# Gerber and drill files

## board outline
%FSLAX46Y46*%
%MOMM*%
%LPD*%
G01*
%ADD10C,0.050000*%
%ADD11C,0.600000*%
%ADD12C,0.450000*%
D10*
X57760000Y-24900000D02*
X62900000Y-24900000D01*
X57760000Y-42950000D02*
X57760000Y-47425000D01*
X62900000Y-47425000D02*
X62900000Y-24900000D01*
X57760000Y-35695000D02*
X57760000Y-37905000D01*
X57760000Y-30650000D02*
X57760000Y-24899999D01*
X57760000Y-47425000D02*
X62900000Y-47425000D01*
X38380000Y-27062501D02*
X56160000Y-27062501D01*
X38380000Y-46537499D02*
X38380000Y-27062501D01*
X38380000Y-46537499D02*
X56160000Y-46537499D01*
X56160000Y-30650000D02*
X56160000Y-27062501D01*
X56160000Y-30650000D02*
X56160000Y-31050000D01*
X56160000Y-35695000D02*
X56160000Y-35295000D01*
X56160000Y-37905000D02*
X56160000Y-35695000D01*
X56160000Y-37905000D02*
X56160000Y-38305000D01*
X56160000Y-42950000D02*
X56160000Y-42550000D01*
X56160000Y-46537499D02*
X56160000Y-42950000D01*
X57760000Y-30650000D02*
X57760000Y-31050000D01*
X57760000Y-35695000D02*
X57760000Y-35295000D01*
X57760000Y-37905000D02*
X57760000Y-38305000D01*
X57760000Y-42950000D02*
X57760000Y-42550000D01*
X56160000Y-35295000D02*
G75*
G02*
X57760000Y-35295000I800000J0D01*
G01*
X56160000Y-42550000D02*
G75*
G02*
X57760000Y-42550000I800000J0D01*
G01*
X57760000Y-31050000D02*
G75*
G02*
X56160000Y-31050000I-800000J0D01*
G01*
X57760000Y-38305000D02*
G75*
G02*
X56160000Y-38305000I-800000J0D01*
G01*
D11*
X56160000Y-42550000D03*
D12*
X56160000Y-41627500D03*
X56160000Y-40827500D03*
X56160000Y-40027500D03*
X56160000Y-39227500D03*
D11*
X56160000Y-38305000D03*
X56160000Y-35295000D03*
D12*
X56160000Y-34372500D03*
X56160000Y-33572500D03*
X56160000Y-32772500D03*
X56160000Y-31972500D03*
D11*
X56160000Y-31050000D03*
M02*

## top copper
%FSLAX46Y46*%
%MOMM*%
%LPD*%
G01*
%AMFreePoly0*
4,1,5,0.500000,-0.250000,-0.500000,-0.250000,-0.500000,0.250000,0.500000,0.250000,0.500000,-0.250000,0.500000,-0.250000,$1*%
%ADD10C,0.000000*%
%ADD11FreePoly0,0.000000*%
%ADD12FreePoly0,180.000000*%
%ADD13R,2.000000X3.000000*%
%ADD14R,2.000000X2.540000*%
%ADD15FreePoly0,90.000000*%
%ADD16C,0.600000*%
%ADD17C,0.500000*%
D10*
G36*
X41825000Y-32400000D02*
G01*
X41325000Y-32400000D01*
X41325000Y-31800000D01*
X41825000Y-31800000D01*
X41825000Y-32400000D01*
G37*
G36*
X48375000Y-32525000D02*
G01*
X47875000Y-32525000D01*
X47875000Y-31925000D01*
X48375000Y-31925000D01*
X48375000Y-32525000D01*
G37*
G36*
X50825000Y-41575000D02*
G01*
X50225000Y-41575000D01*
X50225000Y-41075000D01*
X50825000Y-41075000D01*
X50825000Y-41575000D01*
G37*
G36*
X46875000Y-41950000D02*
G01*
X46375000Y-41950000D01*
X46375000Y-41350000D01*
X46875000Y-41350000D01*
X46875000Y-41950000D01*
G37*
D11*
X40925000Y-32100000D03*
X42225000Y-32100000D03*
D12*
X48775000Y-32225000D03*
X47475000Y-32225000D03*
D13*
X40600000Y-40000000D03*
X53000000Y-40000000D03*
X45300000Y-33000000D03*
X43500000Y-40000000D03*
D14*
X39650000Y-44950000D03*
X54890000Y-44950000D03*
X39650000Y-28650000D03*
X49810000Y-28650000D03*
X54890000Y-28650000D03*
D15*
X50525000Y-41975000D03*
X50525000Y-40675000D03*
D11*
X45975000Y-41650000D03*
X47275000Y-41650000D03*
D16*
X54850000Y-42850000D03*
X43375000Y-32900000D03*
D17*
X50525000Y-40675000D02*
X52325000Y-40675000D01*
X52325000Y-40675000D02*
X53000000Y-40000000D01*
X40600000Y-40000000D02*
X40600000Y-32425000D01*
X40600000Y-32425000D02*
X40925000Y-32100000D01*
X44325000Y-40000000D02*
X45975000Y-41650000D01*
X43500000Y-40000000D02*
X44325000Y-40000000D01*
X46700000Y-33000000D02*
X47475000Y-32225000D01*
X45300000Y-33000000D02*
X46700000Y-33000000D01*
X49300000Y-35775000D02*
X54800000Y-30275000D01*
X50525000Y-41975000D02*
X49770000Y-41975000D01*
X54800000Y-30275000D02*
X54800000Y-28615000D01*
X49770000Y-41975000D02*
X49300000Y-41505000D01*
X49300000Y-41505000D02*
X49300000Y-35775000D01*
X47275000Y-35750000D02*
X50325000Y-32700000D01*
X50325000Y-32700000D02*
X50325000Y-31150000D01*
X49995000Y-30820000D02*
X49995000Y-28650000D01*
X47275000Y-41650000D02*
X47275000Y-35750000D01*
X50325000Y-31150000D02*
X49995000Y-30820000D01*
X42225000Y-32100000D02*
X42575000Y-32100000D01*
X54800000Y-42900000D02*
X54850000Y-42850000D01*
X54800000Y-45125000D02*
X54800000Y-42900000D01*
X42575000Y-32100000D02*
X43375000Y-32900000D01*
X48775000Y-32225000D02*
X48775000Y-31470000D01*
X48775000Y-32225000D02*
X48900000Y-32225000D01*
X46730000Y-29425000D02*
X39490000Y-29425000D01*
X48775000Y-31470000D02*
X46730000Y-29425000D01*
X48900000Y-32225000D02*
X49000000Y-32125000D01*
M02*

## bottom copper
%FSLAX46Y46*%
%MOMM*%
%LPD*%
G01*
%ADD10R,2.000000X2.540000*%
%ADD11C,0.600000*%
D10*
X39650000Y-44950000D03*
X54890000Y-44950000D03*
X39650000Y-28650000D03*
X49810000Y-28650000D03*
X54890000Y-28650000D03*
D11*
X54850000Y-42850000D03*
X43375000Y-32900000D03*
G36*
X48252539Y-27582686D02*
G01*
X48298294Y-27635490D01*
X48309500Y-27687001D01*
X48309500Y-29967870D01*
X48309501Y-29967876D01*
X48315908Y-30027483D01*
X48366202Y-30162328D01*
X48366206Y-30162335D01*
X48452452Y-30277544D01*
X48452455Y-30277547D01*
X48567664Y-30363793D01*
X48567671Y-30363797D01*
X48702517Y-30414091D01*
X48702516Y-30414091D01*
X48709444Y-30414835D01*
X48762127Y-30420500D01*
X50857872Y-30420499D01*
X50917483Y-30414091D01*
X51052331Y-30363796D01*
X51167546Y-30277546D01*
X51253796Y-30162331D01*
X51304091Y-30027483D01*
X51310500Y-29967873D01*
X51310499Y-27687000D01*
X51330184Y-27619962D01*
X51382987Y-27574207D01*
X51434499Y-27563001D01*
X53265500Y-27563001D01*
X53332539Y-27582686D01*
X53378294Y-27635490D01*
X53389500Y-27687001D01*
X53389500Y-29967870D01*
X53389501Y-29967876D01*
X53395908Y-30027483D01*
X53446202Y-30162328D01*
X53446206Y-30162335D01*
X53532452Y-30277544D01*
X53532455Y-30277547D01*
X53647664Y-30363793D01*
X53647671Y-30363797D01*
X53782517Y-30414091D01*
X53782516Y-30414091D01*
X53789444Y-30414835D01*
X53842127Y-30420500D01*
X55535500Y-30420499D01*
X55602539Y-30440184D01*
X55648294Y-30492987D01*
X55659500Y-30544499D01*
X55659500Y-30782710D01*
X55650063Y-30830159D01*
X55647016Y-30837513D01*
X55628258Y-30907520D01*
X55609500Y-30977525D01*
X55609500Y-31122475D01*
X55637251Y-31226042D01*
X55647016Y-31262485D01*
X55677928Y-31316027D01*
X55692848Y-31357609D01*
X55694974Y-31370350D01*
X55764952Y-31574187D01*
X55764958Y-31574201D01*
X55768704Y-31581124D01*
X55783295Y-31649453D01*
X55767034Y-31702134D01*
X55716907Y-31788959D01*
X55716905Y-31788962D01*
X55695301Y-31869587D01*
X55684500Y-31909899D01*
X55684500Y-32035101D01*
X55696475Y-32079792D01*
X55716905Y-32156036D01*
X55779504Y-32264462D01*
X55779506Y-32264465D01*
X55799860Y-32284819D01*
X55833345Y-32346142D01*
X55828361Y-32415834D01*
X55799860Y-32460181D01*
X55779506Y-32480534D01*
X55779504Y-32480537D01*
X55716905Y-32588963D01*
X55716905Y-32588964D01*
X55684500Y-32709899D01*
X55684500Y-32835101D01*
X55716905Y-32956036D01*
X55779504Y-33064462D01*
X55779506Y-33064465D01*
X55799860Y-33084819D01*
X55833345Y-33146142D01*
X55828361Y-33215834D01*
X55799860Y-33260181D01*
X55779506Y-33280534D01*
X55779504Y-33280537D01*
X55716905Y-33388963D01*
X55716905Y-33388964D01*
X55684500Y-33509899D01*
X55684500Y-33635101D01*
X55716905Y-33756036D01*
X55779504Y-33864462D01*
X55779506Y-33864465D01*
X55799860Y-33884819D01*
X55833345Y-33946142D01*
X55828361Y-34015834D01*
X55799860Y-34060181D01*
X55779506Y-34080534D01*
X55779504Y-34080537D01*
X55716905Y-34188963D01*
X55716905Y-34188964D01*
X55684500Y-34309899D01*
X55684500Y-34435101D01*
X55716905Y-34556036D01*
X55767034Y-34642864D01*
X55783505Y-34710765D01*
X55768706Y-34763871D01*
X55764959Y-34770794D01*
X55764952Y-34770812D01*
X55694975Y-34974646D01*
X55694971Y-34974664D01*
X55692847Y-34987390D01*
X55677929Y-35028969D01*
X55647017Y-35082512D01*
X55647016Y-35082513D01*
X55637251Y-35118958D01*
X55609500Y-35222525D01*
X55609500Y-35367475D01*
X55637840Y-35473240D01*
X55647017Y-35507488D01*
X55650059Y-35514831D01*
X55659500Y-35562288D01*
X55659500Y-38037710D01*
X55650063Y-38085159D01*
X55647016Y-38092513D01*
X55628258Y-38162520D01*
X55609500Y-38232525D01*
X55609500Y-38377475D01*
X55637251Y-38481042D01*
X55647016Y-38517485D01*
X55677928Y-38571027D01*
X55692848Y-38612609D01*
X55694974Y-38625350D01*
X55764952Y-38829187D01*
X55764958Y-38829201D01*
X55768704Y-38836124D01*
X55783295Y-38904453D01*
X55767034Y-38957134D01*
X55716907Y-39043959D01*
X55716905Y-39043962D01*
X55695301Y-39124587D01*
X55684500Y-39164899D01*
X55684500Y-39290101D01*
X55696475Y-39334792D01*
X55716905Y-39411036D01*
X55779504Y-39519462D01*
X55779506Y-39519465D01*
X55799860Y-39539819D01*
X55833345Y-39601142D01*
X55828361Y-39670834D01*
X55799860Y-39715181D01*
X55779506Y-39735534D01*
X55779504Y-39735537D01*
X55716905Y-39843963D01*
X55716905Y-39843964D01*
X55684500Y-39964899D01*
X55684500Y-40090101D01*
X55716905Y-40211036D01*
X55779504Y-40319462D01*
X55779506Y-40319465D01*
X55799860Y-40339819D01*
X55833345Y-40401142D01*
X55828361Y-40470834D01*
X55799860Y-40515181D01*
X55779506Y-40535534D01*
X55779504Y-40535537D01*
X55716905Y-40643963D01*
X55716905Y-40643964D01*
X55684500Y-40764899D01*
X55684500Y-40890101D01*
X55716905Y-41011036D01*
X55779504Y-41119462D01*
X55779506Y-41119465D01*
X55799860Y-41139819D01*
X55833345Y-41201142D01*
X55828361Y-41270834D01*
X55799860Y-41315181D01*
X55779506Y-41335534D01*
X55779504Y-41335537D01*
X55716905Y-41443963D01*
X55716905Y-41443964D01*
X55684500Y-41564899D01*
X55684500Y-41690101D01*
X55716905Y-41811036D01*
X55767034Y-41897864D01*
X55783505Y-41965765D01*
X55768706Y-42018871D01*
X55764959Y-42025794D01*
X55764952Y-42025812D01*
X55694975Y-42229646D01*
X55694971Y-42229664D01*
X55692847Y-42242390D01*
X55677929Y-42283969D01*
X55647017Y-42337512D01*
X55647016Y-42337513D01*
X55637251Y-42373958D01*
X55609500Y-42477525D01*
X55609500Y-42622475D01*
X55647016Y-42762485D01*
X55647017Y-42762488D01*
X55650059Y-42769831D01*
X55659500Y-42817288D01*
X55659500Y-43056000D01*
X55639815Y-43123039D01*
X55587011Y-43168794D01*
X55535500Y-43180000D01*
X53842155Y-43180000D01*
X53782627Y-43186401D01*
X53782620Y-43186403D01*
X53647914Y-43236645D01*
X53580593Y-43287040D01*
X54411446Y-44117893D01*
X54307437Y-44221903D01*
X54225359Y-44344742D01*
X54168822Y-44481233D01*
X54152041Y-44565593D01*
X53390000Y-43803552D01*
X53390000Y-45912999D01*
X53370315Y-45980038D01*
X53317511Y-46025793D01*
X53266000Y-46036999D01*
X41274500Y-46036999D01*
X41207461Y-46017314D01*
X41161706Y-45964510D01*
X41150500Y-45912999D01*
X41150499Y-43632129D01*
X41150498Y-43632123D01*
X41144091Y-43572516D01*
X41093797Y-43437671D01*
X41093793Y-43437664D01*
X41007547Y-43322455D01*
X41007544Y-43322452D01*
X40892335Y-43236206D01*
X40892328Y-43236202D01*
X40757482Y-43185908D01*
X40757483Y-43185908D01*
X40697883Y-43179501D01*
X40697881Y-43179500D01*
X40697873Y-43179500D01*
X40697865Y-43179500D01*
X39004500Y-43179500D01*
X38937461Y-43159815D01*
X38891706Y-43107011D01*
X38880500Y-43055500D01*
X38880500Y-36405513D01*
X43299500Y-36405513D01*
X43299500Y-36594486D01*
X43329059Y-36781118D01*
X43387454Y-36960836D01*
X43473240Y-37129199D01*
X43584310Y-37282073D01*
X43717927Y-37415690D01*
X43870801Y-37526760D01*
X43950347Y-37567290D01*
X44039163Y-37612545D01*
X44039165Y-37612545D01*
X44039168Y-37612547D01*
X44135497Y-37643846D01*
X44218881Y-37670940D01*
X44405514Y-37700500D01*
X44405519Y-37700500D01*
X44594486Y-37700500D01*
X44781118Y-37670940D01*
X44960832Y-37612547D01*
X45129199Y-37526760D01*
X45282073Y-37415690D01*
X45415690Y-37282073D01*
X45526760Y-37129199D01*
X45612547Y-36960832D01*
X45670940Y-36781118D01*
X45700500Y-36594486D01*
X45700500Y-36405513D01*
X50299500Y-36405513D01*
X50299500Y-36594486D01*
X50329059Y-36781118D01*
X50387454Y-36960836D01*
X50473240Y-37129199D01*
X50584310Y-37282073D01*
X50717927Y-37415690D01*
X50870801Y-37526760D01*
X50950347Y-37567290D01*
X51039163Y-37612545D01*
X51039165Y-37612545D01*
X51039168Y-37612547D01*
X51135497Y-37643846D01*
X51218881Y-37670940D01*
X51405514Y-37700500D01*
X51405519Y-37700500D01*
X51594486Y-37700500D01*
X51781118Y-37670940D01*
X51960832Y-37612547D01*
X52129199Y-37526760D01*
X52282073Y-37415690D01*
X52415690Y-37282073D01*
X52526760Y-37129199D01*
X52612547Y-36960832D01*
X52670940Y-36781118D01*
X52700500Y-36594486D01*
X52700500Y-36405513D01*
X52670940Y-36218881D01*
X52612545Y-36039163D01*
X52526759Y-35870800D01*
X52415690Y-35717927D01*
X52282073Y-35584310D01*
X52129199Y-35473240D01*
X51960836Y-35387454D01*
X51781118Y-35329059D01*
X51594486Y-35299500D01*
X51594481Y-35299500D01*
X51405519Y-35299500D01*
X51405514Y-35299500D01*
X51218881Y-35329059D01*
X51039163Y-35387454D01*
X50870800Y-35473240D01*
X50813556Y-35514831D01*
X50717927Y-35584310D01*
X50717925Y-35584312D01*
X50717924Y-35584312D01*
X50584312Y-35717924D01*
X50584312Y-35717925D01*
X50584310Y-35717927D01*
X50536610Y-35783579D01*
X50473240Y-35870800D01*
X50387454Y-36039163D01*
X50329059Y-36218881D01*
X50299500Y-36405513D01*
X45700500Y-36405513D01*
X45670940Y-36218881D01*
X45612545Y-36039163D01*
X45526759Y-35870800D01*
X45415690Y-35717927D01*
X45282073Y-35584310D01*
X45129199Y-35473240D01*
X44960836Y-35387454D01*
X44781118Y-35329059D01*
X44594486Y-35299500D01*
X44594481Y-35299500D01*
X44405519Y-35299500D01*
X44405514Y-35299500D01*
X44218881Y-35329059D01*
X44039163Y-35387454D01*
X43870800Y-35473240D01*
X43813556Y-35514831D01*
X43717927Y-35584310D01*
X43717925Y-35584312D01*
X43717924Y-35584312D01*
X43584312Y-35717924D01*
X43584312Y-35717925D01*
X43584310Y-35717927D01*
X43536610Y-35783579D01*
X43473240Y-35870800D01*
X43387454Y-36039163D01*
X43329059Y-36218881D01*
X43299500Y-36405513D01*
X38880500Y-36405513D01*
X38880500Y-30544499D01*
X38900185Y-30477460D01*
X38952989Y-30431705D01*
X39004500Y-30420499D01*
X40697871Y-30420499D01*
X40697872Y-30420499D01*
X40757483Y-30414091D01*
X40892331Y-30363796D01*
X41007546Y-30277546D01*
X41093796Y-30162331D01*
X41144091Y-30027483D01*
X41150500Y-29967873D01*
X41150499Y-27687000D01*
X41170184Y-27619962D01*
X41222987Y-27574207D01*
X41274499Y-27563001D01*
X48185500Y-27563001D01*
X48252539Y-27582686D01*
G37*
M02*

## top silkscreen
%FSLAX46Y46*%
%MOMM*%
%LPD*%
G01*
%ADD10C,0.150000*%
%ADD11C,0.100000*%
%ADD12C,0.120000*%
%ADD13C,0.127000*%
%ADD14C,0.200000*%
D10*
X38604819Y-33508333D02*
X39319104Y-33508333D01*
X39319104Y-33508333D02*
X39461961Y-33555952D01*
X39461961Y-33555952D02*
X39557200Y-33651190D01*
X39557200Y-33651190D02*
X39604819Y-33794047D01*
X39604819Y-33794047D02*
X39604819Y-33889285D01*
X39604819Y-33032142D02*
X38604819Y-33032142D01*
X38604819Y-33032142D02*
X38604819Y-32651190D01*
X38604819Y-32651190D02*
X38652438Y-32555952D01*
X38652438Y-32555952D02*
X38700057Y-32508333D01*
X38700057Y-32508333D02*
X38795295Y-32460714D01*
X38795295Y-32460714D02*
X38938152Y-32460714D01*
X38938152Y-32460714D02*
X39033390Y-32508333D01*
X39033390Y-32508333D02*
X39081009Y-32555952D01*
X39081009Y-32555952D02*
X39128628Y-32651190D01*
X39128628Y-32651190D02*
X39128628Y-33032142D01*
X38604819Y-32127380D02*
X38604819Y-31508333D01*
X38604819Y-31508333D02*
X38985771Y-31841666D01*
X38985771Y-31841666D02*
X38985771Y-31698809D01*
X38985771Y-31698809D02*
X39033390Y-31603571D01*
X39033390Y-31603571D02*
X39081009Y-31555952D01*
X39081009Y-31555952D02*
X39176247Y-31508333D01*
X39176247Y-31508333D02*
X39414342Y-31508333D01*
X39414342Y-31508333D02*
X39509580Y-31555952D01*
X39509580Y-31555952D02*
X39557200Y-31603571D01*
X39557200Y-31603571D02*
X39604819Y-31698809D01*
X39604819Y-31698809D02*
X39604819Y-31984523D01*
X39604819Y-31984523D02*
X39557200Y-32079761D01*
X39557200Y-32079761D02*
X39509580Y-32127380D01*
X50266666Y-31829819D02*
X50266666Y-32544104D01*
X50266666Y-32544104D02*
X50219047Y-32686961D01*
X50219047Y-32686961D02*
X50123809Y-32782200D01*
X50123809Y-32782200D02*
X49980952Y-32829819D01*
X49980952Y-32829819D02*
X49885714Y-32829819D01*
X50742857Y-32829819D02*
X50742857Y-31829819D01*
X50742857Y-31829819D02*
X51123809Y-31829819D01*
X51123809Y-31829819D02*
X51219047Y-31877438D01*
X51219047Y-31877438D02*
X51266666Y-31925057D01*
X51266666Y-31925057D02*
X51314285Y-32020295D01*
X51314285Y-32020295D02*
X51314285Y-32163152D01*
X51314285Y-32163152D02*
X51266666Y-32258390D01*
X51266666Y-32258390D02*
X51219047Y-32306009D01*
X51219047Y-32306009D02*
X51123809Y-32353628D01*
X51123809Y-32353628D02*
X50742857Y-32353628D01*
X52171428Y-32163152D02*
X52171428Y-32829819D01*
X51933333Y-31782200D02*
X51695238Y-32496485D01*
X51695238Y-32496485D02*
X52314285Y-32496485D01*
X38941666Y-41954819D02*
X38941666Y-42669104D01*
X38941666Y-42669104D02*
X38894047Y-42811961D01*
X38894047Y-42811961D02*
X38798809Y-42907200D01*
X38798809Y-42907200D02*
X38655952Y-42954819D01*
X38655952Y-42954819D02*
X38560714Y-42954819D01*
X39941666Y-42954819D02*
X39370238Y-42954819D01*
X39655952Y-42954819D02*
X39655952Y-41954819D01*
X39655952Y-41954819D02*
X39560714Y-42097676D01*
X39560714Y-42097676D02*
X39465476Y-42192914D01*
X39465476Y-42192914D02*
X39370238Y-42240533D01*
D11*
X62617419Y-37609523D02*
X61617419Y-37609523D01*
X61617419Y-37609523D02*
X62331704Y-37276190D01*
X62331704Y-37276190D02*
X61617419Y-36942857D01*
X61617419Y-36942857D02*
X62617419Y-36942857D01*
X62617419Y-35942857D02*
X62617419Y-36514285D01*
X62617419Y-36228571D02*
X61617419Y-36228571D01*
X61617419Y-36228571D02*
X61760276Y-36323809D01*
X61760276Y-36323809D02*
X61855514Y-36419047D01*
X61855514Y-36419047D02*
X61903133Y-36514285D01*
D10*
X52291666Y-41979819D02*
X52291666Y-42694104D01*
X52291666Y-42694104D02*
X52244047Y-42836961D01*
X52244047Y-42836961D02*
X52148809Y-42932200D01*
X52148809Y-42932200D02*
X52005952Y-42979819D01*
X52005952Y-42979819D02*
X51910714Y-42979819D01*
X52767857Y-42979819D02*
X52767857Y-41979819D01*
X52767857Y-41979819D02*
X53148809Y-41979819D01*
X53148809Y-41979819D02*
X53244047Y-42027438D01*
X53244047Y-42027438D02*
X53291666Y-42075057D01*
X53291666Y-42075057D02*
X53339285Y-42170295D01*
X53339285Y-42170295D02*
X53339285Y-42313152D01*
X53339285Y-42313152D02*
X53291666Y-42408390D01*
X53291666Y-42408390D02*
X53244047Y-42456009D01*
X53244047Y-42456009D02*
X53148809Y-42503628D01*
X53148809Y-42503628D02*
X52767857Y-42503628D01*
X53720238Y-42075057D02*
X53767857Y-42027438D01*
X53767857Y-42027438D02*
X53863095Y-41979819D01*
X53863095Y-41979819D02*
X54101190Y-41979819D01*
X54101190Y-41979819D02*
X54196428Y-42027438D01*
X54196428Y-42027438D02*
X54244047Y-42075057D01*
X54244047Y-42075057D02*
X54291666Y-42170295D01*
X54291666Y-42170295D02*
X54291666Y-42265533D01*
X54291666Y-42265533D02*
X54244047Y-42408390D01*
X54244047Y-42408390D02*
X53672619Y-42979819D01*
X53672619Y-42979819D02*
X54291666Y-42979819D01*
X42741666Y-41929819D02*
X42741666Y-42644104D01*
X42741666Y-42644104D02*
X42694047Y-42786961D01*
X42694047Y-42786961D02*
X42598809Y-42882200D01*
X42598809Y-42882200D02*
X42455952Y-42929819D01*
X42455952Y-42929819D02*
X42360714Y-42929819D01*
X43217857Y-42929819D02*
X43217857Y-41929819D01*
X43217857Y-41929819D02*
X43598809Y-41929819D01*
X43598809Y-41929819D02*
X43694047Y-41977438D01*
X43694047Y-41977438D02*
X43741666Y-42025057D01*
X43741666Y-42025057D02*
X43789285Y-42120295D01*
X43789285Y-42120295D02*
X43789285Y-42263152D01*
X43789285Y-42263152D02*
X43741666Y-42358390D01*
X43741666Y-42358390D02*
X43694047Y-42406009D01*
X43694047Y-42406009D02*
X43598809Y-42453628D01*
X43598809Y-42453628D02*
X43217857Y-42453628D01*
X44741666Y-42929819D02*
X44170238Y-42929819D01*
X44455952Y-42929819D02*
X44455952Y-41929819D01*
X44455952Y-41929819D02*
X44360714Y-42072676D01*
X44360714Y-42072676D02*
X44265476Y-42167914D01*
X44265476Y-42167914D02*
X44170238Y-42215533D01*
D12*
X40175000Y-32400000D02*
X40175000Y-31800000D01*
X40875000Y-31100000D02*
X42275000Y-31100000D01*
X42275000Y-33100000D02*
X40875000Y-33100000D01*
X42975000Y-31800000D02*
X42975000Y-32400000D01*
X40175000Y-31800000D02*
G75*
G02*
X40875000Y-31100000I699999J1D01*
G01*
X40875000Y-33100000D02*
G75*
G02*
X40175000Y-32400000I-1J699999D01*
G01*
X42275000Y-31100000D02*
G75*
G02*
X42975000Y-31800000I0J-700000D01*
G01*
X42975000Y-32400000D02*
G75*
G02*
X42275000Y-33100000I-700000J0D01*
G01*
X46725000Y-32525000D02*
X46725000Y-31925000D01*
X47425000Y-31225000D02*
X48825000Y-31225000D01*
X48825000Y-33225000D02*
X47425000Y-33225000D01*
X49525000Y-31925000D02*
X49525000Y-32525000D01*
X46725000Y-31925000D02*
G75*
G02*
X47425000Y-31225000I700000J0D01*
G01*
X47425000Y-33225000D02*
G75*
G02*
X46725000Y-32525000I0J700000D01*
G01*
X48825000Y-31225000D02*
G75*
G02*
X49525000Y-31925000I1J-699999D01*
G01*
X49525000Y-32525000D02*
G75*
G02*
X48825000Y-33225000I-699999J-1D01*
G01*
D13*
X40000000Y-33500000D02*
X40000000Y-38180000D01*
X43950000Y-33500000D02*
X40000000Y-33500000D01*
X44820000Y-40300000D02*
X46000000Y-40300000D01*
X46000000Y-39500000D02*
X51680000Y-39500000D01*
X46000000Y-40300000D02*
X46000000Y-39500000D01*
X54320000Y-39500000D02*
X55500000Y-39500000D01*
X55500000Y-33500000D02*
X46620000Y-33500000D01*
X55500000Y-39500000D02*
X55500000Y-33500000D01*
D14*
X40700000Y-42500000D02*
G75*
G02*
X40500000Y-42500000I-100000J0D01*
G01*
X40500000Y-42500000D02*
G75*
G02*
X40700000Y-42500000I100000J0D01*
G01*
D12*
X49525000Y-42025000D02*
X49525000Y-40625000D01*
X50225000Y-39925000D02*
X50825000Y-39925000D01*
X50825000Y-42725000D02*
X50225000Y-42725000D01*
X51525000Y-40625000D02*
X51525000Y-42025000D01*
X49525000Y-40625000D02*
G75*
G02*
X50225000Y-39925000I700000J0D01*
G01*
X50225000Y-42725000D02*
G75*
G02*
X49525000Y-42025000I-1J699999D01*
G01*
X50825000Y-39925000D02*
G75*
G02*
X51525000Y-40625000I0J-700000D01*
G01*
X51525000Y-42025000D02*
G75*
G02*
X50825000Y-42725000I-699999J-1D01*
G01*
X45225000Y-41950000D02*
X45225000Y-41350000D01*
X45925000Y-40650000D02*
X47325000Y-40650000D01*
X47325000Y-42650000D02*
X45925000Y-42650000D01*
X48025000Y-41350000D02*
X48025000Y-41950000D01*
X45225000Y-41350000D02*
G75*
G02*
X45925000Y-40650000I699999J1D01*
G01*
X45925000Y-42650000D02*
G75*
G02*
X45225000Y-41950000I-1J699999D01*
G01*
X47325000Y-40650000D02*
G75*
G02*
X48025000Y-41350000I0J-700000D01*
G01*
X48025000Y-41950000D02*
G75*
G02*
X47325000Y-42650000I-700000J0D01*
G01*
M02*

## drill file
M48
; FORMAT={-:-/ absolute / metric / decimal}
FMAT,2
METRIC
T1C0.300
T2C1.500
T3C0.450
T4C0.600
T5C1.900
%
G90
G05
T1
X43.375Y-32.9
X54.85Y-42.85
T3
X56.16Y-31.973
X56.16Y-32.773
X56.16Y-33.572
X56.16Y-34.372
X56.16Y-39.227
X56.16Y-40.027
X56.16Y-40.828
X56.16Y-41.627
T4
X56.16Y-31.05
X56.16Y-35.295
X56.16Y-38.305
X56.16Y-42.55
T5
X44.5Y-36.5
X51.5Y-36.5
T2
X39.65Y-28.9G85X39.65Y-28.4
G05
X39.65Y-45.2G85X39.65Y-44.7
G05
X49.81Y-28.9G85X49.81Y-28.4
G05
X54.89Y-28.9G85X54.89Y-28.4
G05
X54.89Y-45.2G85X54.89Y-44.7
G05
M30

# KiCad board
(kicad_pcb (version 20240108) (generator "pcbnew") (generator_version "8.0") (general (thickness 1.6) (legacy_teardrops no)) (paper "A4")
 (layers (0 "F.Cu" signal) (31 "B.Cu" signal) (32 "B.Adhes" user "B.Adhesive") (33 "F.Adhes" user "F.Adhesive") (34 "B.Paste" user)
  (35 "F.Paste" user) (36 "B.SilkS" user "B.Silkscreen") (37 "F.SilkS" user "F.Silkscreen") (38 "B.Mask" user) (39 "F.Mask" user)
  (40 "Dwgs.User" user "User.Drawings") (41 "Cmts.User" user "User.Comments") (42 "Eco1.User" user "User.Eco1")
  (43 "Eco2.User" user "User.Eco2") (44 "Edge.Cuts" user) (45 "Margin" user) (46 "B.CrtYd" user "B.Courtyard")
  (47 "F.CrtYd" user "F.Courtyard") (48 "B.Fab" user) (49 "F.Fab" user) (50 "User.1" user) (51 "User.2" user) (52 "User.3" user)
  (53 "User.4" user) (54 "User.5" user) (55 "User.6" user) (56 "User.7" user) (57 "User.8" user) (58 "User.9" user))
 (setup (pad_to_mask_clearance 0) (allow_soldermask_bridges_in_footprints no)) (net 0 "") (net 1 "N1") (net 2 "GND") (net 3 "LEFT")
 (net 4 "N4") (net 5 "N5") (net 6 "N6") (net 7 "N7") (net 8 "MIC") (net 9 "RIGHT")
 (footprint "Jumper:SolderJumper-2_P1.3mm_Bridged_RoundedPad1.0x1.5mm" (layer "F.Cu") (at 41.575 32.1)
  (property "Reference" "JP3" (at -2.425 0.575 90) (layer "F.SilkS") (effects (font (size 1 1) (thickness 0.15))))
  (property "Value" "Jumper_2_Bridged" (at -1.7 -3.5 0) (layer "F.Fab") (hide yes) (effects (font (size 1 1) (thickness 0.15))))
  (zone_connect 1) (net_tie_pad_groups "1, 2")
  (fp_poly (pts (xy 0.25 -0.3) (xy -0.25 -0.3) (xy -0.25 0.3) (xy 0.25 0.3)) (stroke (width 0) (type solid)) (fill solid) (layer "F.Cu"))
  (fp_line (start -1.4 0.3) (end -1.4 -0.3) (stroke (width 0.12) (type solid)) (layer "F.SilkS"))
  (fp_line (start -0.7 -1) (end 0.7 -1) (stroke (width 0.12) (type solid)) (layer "F.SilkS"))
  (fp_line (start 0.7 1) (end -0.7 1) (stroke (width 0.12) (type solid)) (layer "F.SilkS"))
  (fp_line (start 1.4 -0.3) (end 1.4 0.3) (stroke (width 0.12) (type solid)) (layer "F.SilkS"))
  (fp_arc (start -1.4 -0.3) (mid -1.194975 -0.794975) (end -0.7 -1) (stroke (width 0.12) (type solid)) (layer "F.SilkS"))
  (fp_arc (start -0.7 1) (mid -1.194975 0.794975) (end -1.4 0.3) (stroke (width 0.12) (type solid)) (layer "F.SilkS"))
  (fp_arc (start 0.7 -1) (mid 1.194975 -0.794975) (end 1.4 -0.3) (stroke (width 0.12) (type solid)) (layer "F.SilkS"))
  (fp_arc (start 1.4 0.3) (mid 1.194975 0.794975) (end 0.7 1) (stroke (width 0.12) (type solid)) (layer "F.SilkS"))
  (pad "1" smd custom (at -0.65 0) (size 1 0.5) (layers "F.Cu" "F.Mask") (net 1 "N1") (zone_connect 2) (thermal_bridge_angle 45)
   (options (clearance outline) (anchor rect)) (primitives))
  (pad "2" smd custom (at 0.65 0) (size 1 0.5) (layers "F.Cu" "F.Mask") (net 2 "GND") (zone_connect 2) (thermal_bridge_angle 45)
   (options (clearance outline) (anchor rect)) (primitives)))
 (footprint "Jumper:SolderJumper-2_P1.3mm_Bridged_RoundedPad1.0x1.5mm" (layer "F.Cu") (at 48.125 32.225 180)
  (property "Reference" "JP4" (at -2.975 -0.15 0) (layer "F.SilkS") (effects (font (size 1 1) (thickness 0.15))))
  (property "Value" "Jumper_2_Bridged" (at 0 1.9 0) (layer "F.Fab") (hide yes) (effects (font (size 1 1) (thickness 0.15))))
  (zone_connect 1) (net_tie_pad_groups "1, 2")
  (fp_poly (pts (xy 0.25 -0.3) (xy -0.25 -0.3) (xy -0.25 0.3) (xy 0.25 0.3)) (stroke (width 0) (type solid)) (fill solid) (layer "F.Cu"))
  (fp_line (start 1.4 -0.3) (end 1.4 0.3) (stroke (width 0.12) (type solid)) (layer "F.SilkS"))
  (fp_line (start 0.7 1) (end -0.7 1) (stroke (width 0.12) (type solid)) (layer "F.SilkS"))
  (fp_line (start -0.7 -1) (end 0.7 -1) (stroke (width 0.12) (type solid)) (layer "F.SilkS"))
  (fp_line (start -1.4 0.3) (end -1.4 -0.3) (stroke (width 0.12) (type solid)) (layer "F.SilkS"))
  (fp_arc (start 1.4 0.3) (mid 1.194975 0.794975) (end 0.7 1) (stroke (width 0.12) (type solid)) (layer "F.SilkS"))
  (fp_arc (start 0.7 -1) (mid 1.194975 -0.794975) (end 1.4 -0.3) (stroke (width 0.12) (type solid)) (layer "F.SilkS"))
  (fp_arc (start -0.7 1) (mid -1.194975 0.794975) (end -1.4 0.3) (stroke (width 0.12) (type solid)) (layer "F.SilkS"))
  (fp_arc (start -1.4 -0.3) (mid -1.194975 -0.794975) (end -0.7 -1) (stroke (width 0.12) (type solid)) (layer "F.SilkS"))
  (pad "1" smd custom (at -0.65 0 180) (size 1 0.5) (layers "F.Cu" "F.Mask") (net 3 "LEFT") (zone_connect 2) (thermal_bridge_angle 45)
   (options (clearance outline) (anchor rect)) (primitives))
  (pad "2" smd custom (at 0.65 0 180) (size 1 0.5) (layers "F.Cu" "F.Mask") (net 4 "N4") (zone_connect 2) (thermal_bridge_angle 45)
   (options (clearance outline) (anchor rect)) (primitives)))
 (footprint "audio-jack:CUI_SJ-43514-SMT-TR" (layer "F.Cu") (at 40.6 40)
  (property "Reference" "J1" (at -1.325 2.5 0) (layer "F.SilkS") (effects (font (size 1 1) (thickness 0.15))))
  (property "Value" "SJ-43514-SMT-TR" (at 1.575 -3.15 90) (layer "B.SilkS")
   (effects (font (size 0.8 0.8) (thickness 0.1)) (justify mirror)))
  (fp_line (start -0.6 -6.5) (end -0.6 -1.82) (stroke (width 0.127) (type solid)) (layer "F.SilkS"))
  (fp_line (start 3.35 -6.5) (end -0.6 -6.5) (stroke (width 0.127) (type solid)) (layer "F.SilkS"))
  (fp_line (start 4.22 0.3) (end 5.4 0.3) (stroke (width 0.127) (type solid)) (layer "F.SilkS"))
  (fp_line (start 5.4 -0.5) (end 11.08 -0.5) (stroke (width 0.127) (type solid)) (layer "F.SilkS"))
  (fp_line (start 5.4 0.3) (end 5.4 -0.5) (stroke (width 0.127) (type solid)) (layer "F.SilkS"))
  (fp_line (start 13.72 -0.5) (end 14.9 -0.5) (stroke (width 0.127) (type solid)) (layer "F.SilkS"))
  (fp_line (start 14.9 -6.5) (end 6.02 -6.5) (stroke (width 0.127) (type solid)) (layer "F.SilkS"))
  (fp_line (start 14.9 -0.5) (end 14.9 -6.5) (stroke (width 0.127) (type solid)) (layer "F.SilkS"))
  (fp_circle (center 0 2.5) (end 0.1 2.5) (stroke (width 0.2) (type solid)) (fill none) (layer "F.SilkS"))
  (pad "" np_thru_hole circle (at 3.9 -3.5) (size 1.9 1.9) (drill 1.9) (layers "*.Cu" "*.Mask"))
  (pad "" np_thru_hole circle (at 10.9 -3.5) (size 1.9 1.9) (drill 1.9) (layers "*.Cu" "*.Mask"))
  (pad "1" smd rect (at 0 0) (size 2 3) (layers "F.Cu" "F.Paste" "F.Mask") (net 1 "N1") (solder_mask_margin 0.102))
  (pad "2" smd rect (at 12.4 0) (size 2 3) (layers "F.Cu" "F.Paste" "F.Mask") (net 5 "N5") (solder_mask_margin 0.102))
  (pad "3" smd rect (at 4.7 -7) (size 2 3) (layers "F.Cu" "F.Paste" "F.Mask") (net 4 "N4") (solder_mask_margin 0.102))
  (pad "4" smd rect (at 2.9 0) (size 2 3) (layers "F.Cu" "F.Paste" "F.Mask") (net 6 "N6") (solder_mask_margin 0.102)))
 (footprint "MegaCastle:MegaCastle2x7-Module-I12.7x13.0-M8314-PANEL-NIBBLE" (layer "F.Cu") (at 47.27 36.8 90)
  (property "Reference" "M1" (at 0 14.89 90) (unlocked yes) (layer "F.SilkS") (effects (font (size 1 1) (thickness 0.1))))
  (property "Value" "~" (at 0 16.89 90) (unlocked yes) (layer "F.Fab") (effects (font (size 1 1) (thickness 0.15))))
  (fp_line (start 9.737499 -8.89) (end 9.737499 8.89) (stroke (width 0.05) (type default)) (layer "Edge.Cuts"))
  (fp_line (start -9.737499 -8.89) (end 9.737499 -8.89) (stroke (width 0.05) (type default)) (layer "Edge.Cuts"))
  (fp_line (start -9.737499 -8.89) (end -9.737499 8.89) (stroke (width 0.05) (type default)) (layer "Edge.Cuts"))
  (fp_line (start 6.15 8.89) (end 9.737499 8.89) (stroke (width 0.05) (type default)) (layer "Edge.Cuts"))
  (fp_line (start 6.15 8.89) (end 5.75 8.89) (stroke (width 0.05) (type default)) (layer "Edge.Cuts"))
  (fp_line (start 1.105 8.89) (end 1.505 8.89) (stroke (width 0.05) (type default)) (layer "Edge.Cuts"))
  (fp_line (start -1.105 8.89) (end 1.105 8.89) (stroke (width 0.05) (type default)) (layer "Edge.Cuts"))
  (fp_line (start -1.105 8.89) (end -1.505 8.89) (stroke (width 0.05) (type default)) (layer "Edge.Cuts"))
  (fp_line (start -6.15 8.89) (end -5.75 8.89) (stroke (width 0.05) (type default)) (layer "Edge.Cuts"))
  (fp_line (start -9.737499 8.89) (end -6.15 8.89) (stroke (width 0.05) (type default)) (layer "Edge.Cuts"))
  (fp_line (start 6.15 10.49) (end 5.75 10.49) (stroke (width 0.05) (type default)) (layer "Edge.Cuts"))
  (fp_line (start 1.105 10.49) (end 1.505 10.49) (stroke (width 0.05) (type default)) (layer "Edge.Cuts"))
  (fp_line (start -1.105 10.49) (end -1.505 10.49) (stroke (width 0.05) (type default)) (layer "Edge.Cuts"))
  (fp_line (start -6.15 10.49) (end -5.75 10.49) (stroke (width 0.05) (type default)) (layer "Edge.Cuts"))
  (fp_arc (start 1.505 8.89) (mid 2.305 9.69) (end 1.505 10.49) (stroke (width 0.05) (type default)) (layer "Edge.Cuts"))
  (fp_arc (start -5.75 8.89) (mid -4.95 9.69) (end -5.75 10.49) (stroke (width 0.05) (type default)) (layer "Edge.Cuts"))
  (fp_arc (start 5.75 10.49) (mid 4.95 9.69) (end 5.75 8.89) (stroke (width 0.05) (type default)) (layer "Edge.Cuts"))
  (fp_arc (start -1.505 10.49) (mid -2.305 9.69) (end -1.505 8.89) (stroke (width 0.05) (type default)) (layer "Edge.Cuts"))
  (pad "" np_thru_hole circle (at -5.75 8.89 90) (size 0.6 0.6) (drill 0.6) (layers "F&B.Cu" "Edge.Cuts"))
  (pad "" np_thru_hole circle (at -4.8275 8.89 90) (size 0.45 0.45) (drill 0.45) (layers "F&B.Cu" "Edge.Cuts"))
  (pad "" np_thru_hole circle (at -4.0275 8.89 90) (size 0.45 0.45) (drill 0.45) (layers "F&B.Cu" "Edge.Cuts"))
  (pad "" np_thru_hole circle (at -3.2275 8.89 90) (size 0.45 0.45) (drill 0.45) (layers "F&B.Cu" "Edge.Cuts"))
  (pad "" np_thru_hole circle (at -2.4275 8.89 90) (size 0.45 0.45) (drill 0.45) (layers "F&B.Cu" "Edge.Cuts"))
  (pad "" np_thru_hole circle (at -1.505 8.89 90) (size 0.6 0.6) (drill 0.6) (layers "F&B.Cu" "Edge.Cuts"))
  (pad "" np_thru_hole circle (at 1.505 8.89 90) (size 0.6 0.6) (drill 0.6) (layers "F&B.Cu" "Edge.Cuts"))
  (pad "" np_thru_hole circle (at 2.4275 8.89 90) (size 0.45 0.45) (drill 0.45) (layers "F&B.Cu" "Edge.Cuts"))
  (pad "" np_thru_hole circle (at 3.2275 8.89 90) (size 0.45 0.45) (drill 0.45) (layers "F&B.Cu" "Edge.Cuts"))
  (pad "" np_thru_hole circle (at 4.0275 8.89 90) (size 0.45 0.45) (drill 0.45) (layers "F&B.Cu" "Edge.Cuts"))
  (pad "" np_thru_hole circle (at 4.8275 8.89 90) (size 0.45 0.45) (drill 0.45) (layers "F&B.Cu" "Edge.Cuts"))
  (pad "" np_thru_hole circle (at 5.75 8.89 90) (size 0.6 0.6) (drill 0.6) (layers "F&B.Cu" "Edge.Cuts"))
  (pad "1" thru_hole rect (at -8.15 -7.62 90) (size 2.54 2) (drill oval 2 1.5) (layers "*.Cu" "*.Mask") (remove_unused_layers no)
   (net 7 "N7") (thermal_bridge_angle 45))
  (pad "7" thru_hole rect (at -8.15 7.62 90) (size 2.54 2) (drill oval 2 1.5) (layers "*.Cu" "*.Mask") (remove_unused_layers no)
   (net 2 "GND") (thermal_bridge_angle 45))
  (pad "8" thru_hole rect (at 8.15 -7.62 90) (size 2.54 2) (drill oval 2 1.5) (layers "*.Cu" "*.Mask") (remove_unused_layers no)
   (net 3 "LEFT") (thermal_bridge_angle 45))
  (pad "12" thru_hole rect (at 8.15 2.54 90) (size 2.54 2) (drill oval 2 1.5) (layers "*.Cu" "*.Mask") (remove_unused_layers no)
   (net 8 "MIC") (thermal_bridge_angle 45))
  (pad "14" thru_hole rect (at 8.15 7.62 90) (size 2.54 2) (drill oval 2 1.5) (layers "*.Cu" "*.Mask") (remove_unused_layers no)
   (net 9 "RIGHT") (thermal_bridge_angle 45))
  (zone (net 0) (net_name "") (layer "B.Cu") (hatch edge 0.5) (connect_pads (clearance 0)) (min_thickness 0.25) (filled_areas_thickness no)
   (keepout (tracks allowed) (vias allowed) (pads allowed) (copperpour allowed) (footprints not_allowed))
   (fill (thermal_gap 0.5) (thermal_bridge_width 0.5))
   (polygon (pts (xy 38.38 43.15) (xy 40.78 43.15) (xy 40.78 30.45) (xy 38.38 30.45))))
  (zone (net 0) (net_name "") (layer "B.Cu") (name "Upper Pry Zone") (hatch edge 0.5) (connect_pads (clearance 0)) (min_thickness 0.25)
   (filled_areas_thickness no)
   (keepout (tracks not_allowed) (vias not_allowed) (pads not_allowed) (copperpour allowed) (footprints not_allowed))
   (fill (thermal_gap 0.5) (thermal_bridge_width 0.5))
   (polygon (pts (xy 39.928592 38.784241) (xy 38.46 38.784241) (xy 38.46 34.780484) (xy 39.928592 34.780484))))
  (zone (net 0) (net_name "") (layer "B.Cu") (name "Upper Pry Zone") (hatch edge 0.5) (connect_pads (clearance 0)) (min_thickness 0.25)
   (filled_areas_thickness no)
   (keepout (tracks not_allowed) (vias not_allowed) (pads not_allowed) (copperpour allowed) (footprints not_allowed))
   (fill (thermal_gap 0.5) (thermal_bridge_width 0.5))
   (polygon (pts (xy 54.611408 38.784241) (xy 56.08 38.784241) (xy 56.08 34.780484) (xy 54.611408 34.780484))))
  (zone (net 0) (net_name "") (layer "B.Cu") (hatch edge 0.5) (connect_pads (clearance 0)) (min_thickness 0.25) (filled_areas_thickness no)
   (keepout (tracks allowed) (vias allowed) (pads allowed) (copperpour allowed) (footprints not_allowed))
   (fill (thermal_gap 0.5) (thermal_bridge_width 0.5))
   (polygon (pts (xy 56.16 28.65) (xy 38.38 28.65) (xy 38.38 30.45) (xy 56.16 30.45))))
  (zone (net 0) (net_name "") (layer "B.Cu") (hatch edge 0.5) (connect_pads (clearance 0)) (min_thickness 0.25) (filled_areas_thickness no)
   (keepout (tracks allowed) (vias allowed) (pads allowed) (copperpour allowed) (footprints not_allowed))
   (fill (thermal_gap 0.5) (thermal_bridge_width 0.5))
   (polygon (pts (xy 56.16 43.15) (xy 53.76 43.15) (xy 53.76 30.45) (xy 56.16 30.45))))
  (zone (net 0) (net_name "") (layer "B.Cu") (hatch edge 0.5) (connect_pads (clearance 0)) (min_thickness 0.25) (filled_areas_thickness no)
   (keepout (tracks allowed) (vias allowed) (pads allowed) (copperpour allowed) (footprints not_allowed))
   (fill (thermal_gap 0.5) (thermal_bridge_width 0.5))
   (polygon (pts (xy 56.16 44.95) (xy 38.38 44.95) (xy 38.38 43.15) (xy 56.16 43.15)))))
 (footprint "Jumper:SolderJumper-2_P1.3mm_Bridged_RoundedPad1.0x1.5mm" (layer "F.Cu") (at 50.525 41.325 90)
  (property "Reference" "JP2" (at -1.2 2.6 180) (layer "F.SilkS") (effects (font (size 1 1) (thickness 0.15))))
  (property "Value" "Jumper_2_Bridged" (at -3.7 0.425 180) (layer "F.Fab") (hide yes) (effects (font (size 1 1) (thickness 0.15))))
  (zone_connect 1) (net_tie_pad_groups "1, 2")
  (fp_poly (pts (xy 0.25 -0.3) (xy -0.25 -0.3) (xy -0.25 0.3) (xy 0.25 0.3)) (stroke (width 0) (type solid)) (fill solid) (layer "F.Cu"))
  (fp_line (start -0.7 -1) (end 0.7 -1) (stroke (width 0.12) (type solid)) (layer "F.SilkS"))
  (fp_line (start 1.4 -0.3) (end 1.4 0.3) (stroke (width 0.12) (type solid)) (layer "F.SilkS"))
  (fp_line (start -1.4 0.3) (end -1.4 -0.3) (stroke (width 0.12) (type solid)) (layer "F.SilkS"))
  (fp_line (start 0.7 1) (end -0.7 1) (stroke (width 0.12) (type solid)) (layer "F.SilkS"))
  (fp_arc (start 0.7 -1) (mid 1.194975 -0.794975) (end 1.4 -0.3) (stroke (width 0.12) (type solid)) (layer "F.SilkS"))
  (fp_arc (start -1.4 -0.3) (mid -1.194975 -0.794975) (end -0.7 -1) (stroke (width 0.12) (type solid)) (layer "F.SilkS"))
  (fp_arc (start 1.4 0.3) (mid 1.194975 0.794975) (end 0.7 1) (stroke (width 0.12) (type solid)) (layer "F.SilkS"))
  (fp_arc (start -0.7 1) (mid -1.194975 0.794975) (end -1.4 0.3) (stroke (width 0.12) (type solid)) (layer "F.SilkS"))
  (pad "1" smd custom (at -0.65 0 90) (size 1 0.5) (layers "F.Cu" "F.Mask") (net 9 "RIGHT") (zone_connect 2) (thermal_bridge_angle 45)
   (options (clearance outline) (anchor rect)) (primitives))
  (pad "2" smd custom (at 0.65 0 90) (size 1 0.5) (layers "F.Cu" "F.Mask") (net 5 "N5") (zone_connect 2) (thermal_bridge_angle 45)
   (options (clearance outline) (anchor rect)) (primitives)))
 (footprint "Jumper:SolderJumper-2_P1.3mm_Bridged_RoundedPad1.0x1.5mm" (layer "F.Cu") (at 46.625 41.65)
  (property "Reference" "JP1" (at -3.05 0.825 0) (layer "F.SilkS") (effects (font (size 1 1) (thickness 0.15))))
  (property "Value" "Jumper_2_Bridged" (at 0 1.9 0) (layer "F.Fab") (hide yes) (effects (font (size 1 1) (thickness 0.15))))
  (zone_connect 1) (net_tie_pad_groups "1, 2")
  (fp_poly (pts (xy 0.25 -0.3) (xy -0.25 -0.3) (xy -0.25 0.3) (xy 0.25 0.3)) (stroke (width 0) (type solid)) (fill solid) (layer "F.Cu"))
  (fp_line (start -1.4 0.3) (end -1.4 -0.3) (stroke (width 0.12) (type solid)) (layer "F.SilkS"))
  (fp_line (start -0.7 -1) (end 0.7 -1) (stroke (width 0.12) (type solid)) (layer "F.SilkS"))
  (fp_line (start 0.7 1) (end -0.7 1) (stroke (width 0.12) (type solid)) (layer "F.SilkS"))
  (fp_line (start 1.4 -0.3) (end 1.4 0.3) (stroke (width 0.12) (type solid)) (layer "F.SilkS"))
  (fp_arc (start -1.4 -0.3) (mid -1.194975 -0.794975) (end -0.7 -1) (stroke (width 0.12) (type solid)) (layer "F.SilkS"))
  (fp_arc (start -0.7 1) (mid -1.194975 0.794975) (end -1.4 0.3) (stroke (width 0.12) (type solid)) (layer "F.SilkS"))
  (fp_arc (start 0.7 -1) (mid 1.194975 -0.794975) (end 1.4 -0.3) (stroke (width 0.12) (type solid)) (layer "F.SilkS"))
  (fp_arc (start 1.4 0.3) (mid 1.194975 0.794975) (end 0.7 1) (stroke (width 0.12) (type solid)) (layer "F.SilkS"))
  (pad "1" smd custom (at -0.65 0) (size 1 0.5) (layers "F.Cu" "F.Mask") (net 6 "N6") (zone_connect 2) (thermal_bridge_angle 45)
   (options (clearance outline) (anchor rect)) (primitives))
  (pad "2" smd custom (at 0.65 0) (size 1 0.5) (layers "F.Cu" "F.Mask") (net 8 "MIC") (zone_connect 2) (thermal_bridge_angle 45)
   (options (clearance outline) (anchor rect)) (primitives)))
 (gr_line (start 57.76 24.9) (end 62.9 24.9) (stroke (width 0.05) (type default)) (layer "Edge.Cuts"))
 (gr_line (start 57.76 42.95) (end 57.76 47.425) (stroke (width 0.05) (type default)) (layer "Edge.Cuts"))
 (gr_line (start 62.9 47.425) (end 62.9 24.9) (stroke (width 0.05) (type default)) (layer "Edge.Cuts"))
 (gr_line (start 57.76 35.695) (end 57.76 37.905) (stroke (width 0.05) (type default)) (layer "Edge.Cuts"))
 (gr_line (start 57.76 30.65) (end 57.76 24.899999) (stroke (width 0.05) (type default)) (layer "Edge.Cuts"))
 (gr_line (start 57.76 47.425) (end 62.9 47.425) (stroke (width 0.05) (type default)) (layer "Edge.Cuts"))
 (segment (start 50.525 40.675) (end 52.325 40.675) (width 0.5) (layer "F.Cu") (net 5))
 (segment (start 52.325 40.675) (end 53 40) (width 0.5) (layer "F.Cu") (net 5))
 (segment (start 40.6 40) (end 40.6 32.425) (width 0.5) (layer "F.Cu") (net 1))
 (segment (start 40.6 32.425) (end 40.925 32.1) (width 0.5) (layer "F.Cu") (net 1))
 (segment (start 44.325 40) (end 45.975 41.65) (width 0.5) (layer "F.Cu") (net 6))
 (segment (start 43.5 40) (end 44.325 40) (width 0.5) (layer "F.Cu") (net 6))
 (segment (start 46.7 33) (end 47.475 32.225) (width 0.5) (layer "F.Cu") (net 4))
 (segment (start 45.3 33) (end 46.7 33) (width 0.5) (layer "F.Cu") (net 4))
 (segment (start 49.3 35.775) (end 54.8 30.275) (width 0.5) (layer "F.Cu") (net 9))
 (segment (start 50.525 41.975) (end 49.77 41.975) (width 0.5) (layer "F.Cu") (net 9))
 (segment (start 54.8 30.275) (end 54.8 28.615) (width 0.5) (layer "F.Cu") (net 9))
 (segment (start 49.77 41.975) (end 49.3 41.505) (width 0.5) (layer "F.Cu") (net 9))
 (segment (start 49.3 41.505) (end 49.3 35.775) (width 0.5) (layer "F.Cu") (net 9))
 (segment (start 47.275 35.75) (end 50.325 32.7) (width 0.5) (layer "F.Cu") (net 8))
 (segment (start 50.325 32.7) (end 50.325 31.15) (width 0.5) (layer "F.Cu") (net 8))
 (segment (start 49.995 30.82) (end 49.995 28.65) (width 0.5) (layer "F.Cu") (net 8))
 (segment (start 47.275 41.65) (end 47.275 35.75) (width 0.5) (layer "F.Cu") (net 8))
 (segment (start 50.325 31.15) (end 49.995 30.82) (width 0.5) (layer "F.Cu") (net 8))
 (segment (start 42.225 32.1) (end 42.575 32.1) (width 0.5) (layer "F.Cu") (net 2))
 (segment (start 54.8 42.9) (end 54.85 42.85) (width 0.5) (layer "F.Cu") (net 2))
 (segment (start 54.8 45.125) (end 54.8 42.9) (width 0.5) (layer "F.Cu") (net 2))
 (segment (start 42.575 32.1) (end 43.375 32.9) (width 0.5) (layer "F.Cu") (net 2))
 (via (at 54.85 42.85) (size 0.6) (drill 0.3) (layers "F.Cu" "B.Cu") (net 2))
 (via (at 43.375 32.9) (size 0.6) (drill 0.3) (layers "F.Cu" "B.Cu") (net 2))
 (segment (start 48.775 32.225) (end 48.775 31.47) (width 0.5) (layer "F.Cu") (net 3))
 (segment (start 48.775 32.225) (end 48.9 32.225) (width 0.5) (layer "F.Cu") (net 3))
 (segment (start 46.73 29.425) (end 39.49 29.425) (width 0.5) (layer "F.Cu") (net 3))
 (segment (start 48.775 31.47) (end 46.73 29.425) (width 0.5) (layer "F.Cu") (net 3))
 (segment (start 48.9 32.225) (end 49 32.125) (width 0.5) (layer "F.Cu") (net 3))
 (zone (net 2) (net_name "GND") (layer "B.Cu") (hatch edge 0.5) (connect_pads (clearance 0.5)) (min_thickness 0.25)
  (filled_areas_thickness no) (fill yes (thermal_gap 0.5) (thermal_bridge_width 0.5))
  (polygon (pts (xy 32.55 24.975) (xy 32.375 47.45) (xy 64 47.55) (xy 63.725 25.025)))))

